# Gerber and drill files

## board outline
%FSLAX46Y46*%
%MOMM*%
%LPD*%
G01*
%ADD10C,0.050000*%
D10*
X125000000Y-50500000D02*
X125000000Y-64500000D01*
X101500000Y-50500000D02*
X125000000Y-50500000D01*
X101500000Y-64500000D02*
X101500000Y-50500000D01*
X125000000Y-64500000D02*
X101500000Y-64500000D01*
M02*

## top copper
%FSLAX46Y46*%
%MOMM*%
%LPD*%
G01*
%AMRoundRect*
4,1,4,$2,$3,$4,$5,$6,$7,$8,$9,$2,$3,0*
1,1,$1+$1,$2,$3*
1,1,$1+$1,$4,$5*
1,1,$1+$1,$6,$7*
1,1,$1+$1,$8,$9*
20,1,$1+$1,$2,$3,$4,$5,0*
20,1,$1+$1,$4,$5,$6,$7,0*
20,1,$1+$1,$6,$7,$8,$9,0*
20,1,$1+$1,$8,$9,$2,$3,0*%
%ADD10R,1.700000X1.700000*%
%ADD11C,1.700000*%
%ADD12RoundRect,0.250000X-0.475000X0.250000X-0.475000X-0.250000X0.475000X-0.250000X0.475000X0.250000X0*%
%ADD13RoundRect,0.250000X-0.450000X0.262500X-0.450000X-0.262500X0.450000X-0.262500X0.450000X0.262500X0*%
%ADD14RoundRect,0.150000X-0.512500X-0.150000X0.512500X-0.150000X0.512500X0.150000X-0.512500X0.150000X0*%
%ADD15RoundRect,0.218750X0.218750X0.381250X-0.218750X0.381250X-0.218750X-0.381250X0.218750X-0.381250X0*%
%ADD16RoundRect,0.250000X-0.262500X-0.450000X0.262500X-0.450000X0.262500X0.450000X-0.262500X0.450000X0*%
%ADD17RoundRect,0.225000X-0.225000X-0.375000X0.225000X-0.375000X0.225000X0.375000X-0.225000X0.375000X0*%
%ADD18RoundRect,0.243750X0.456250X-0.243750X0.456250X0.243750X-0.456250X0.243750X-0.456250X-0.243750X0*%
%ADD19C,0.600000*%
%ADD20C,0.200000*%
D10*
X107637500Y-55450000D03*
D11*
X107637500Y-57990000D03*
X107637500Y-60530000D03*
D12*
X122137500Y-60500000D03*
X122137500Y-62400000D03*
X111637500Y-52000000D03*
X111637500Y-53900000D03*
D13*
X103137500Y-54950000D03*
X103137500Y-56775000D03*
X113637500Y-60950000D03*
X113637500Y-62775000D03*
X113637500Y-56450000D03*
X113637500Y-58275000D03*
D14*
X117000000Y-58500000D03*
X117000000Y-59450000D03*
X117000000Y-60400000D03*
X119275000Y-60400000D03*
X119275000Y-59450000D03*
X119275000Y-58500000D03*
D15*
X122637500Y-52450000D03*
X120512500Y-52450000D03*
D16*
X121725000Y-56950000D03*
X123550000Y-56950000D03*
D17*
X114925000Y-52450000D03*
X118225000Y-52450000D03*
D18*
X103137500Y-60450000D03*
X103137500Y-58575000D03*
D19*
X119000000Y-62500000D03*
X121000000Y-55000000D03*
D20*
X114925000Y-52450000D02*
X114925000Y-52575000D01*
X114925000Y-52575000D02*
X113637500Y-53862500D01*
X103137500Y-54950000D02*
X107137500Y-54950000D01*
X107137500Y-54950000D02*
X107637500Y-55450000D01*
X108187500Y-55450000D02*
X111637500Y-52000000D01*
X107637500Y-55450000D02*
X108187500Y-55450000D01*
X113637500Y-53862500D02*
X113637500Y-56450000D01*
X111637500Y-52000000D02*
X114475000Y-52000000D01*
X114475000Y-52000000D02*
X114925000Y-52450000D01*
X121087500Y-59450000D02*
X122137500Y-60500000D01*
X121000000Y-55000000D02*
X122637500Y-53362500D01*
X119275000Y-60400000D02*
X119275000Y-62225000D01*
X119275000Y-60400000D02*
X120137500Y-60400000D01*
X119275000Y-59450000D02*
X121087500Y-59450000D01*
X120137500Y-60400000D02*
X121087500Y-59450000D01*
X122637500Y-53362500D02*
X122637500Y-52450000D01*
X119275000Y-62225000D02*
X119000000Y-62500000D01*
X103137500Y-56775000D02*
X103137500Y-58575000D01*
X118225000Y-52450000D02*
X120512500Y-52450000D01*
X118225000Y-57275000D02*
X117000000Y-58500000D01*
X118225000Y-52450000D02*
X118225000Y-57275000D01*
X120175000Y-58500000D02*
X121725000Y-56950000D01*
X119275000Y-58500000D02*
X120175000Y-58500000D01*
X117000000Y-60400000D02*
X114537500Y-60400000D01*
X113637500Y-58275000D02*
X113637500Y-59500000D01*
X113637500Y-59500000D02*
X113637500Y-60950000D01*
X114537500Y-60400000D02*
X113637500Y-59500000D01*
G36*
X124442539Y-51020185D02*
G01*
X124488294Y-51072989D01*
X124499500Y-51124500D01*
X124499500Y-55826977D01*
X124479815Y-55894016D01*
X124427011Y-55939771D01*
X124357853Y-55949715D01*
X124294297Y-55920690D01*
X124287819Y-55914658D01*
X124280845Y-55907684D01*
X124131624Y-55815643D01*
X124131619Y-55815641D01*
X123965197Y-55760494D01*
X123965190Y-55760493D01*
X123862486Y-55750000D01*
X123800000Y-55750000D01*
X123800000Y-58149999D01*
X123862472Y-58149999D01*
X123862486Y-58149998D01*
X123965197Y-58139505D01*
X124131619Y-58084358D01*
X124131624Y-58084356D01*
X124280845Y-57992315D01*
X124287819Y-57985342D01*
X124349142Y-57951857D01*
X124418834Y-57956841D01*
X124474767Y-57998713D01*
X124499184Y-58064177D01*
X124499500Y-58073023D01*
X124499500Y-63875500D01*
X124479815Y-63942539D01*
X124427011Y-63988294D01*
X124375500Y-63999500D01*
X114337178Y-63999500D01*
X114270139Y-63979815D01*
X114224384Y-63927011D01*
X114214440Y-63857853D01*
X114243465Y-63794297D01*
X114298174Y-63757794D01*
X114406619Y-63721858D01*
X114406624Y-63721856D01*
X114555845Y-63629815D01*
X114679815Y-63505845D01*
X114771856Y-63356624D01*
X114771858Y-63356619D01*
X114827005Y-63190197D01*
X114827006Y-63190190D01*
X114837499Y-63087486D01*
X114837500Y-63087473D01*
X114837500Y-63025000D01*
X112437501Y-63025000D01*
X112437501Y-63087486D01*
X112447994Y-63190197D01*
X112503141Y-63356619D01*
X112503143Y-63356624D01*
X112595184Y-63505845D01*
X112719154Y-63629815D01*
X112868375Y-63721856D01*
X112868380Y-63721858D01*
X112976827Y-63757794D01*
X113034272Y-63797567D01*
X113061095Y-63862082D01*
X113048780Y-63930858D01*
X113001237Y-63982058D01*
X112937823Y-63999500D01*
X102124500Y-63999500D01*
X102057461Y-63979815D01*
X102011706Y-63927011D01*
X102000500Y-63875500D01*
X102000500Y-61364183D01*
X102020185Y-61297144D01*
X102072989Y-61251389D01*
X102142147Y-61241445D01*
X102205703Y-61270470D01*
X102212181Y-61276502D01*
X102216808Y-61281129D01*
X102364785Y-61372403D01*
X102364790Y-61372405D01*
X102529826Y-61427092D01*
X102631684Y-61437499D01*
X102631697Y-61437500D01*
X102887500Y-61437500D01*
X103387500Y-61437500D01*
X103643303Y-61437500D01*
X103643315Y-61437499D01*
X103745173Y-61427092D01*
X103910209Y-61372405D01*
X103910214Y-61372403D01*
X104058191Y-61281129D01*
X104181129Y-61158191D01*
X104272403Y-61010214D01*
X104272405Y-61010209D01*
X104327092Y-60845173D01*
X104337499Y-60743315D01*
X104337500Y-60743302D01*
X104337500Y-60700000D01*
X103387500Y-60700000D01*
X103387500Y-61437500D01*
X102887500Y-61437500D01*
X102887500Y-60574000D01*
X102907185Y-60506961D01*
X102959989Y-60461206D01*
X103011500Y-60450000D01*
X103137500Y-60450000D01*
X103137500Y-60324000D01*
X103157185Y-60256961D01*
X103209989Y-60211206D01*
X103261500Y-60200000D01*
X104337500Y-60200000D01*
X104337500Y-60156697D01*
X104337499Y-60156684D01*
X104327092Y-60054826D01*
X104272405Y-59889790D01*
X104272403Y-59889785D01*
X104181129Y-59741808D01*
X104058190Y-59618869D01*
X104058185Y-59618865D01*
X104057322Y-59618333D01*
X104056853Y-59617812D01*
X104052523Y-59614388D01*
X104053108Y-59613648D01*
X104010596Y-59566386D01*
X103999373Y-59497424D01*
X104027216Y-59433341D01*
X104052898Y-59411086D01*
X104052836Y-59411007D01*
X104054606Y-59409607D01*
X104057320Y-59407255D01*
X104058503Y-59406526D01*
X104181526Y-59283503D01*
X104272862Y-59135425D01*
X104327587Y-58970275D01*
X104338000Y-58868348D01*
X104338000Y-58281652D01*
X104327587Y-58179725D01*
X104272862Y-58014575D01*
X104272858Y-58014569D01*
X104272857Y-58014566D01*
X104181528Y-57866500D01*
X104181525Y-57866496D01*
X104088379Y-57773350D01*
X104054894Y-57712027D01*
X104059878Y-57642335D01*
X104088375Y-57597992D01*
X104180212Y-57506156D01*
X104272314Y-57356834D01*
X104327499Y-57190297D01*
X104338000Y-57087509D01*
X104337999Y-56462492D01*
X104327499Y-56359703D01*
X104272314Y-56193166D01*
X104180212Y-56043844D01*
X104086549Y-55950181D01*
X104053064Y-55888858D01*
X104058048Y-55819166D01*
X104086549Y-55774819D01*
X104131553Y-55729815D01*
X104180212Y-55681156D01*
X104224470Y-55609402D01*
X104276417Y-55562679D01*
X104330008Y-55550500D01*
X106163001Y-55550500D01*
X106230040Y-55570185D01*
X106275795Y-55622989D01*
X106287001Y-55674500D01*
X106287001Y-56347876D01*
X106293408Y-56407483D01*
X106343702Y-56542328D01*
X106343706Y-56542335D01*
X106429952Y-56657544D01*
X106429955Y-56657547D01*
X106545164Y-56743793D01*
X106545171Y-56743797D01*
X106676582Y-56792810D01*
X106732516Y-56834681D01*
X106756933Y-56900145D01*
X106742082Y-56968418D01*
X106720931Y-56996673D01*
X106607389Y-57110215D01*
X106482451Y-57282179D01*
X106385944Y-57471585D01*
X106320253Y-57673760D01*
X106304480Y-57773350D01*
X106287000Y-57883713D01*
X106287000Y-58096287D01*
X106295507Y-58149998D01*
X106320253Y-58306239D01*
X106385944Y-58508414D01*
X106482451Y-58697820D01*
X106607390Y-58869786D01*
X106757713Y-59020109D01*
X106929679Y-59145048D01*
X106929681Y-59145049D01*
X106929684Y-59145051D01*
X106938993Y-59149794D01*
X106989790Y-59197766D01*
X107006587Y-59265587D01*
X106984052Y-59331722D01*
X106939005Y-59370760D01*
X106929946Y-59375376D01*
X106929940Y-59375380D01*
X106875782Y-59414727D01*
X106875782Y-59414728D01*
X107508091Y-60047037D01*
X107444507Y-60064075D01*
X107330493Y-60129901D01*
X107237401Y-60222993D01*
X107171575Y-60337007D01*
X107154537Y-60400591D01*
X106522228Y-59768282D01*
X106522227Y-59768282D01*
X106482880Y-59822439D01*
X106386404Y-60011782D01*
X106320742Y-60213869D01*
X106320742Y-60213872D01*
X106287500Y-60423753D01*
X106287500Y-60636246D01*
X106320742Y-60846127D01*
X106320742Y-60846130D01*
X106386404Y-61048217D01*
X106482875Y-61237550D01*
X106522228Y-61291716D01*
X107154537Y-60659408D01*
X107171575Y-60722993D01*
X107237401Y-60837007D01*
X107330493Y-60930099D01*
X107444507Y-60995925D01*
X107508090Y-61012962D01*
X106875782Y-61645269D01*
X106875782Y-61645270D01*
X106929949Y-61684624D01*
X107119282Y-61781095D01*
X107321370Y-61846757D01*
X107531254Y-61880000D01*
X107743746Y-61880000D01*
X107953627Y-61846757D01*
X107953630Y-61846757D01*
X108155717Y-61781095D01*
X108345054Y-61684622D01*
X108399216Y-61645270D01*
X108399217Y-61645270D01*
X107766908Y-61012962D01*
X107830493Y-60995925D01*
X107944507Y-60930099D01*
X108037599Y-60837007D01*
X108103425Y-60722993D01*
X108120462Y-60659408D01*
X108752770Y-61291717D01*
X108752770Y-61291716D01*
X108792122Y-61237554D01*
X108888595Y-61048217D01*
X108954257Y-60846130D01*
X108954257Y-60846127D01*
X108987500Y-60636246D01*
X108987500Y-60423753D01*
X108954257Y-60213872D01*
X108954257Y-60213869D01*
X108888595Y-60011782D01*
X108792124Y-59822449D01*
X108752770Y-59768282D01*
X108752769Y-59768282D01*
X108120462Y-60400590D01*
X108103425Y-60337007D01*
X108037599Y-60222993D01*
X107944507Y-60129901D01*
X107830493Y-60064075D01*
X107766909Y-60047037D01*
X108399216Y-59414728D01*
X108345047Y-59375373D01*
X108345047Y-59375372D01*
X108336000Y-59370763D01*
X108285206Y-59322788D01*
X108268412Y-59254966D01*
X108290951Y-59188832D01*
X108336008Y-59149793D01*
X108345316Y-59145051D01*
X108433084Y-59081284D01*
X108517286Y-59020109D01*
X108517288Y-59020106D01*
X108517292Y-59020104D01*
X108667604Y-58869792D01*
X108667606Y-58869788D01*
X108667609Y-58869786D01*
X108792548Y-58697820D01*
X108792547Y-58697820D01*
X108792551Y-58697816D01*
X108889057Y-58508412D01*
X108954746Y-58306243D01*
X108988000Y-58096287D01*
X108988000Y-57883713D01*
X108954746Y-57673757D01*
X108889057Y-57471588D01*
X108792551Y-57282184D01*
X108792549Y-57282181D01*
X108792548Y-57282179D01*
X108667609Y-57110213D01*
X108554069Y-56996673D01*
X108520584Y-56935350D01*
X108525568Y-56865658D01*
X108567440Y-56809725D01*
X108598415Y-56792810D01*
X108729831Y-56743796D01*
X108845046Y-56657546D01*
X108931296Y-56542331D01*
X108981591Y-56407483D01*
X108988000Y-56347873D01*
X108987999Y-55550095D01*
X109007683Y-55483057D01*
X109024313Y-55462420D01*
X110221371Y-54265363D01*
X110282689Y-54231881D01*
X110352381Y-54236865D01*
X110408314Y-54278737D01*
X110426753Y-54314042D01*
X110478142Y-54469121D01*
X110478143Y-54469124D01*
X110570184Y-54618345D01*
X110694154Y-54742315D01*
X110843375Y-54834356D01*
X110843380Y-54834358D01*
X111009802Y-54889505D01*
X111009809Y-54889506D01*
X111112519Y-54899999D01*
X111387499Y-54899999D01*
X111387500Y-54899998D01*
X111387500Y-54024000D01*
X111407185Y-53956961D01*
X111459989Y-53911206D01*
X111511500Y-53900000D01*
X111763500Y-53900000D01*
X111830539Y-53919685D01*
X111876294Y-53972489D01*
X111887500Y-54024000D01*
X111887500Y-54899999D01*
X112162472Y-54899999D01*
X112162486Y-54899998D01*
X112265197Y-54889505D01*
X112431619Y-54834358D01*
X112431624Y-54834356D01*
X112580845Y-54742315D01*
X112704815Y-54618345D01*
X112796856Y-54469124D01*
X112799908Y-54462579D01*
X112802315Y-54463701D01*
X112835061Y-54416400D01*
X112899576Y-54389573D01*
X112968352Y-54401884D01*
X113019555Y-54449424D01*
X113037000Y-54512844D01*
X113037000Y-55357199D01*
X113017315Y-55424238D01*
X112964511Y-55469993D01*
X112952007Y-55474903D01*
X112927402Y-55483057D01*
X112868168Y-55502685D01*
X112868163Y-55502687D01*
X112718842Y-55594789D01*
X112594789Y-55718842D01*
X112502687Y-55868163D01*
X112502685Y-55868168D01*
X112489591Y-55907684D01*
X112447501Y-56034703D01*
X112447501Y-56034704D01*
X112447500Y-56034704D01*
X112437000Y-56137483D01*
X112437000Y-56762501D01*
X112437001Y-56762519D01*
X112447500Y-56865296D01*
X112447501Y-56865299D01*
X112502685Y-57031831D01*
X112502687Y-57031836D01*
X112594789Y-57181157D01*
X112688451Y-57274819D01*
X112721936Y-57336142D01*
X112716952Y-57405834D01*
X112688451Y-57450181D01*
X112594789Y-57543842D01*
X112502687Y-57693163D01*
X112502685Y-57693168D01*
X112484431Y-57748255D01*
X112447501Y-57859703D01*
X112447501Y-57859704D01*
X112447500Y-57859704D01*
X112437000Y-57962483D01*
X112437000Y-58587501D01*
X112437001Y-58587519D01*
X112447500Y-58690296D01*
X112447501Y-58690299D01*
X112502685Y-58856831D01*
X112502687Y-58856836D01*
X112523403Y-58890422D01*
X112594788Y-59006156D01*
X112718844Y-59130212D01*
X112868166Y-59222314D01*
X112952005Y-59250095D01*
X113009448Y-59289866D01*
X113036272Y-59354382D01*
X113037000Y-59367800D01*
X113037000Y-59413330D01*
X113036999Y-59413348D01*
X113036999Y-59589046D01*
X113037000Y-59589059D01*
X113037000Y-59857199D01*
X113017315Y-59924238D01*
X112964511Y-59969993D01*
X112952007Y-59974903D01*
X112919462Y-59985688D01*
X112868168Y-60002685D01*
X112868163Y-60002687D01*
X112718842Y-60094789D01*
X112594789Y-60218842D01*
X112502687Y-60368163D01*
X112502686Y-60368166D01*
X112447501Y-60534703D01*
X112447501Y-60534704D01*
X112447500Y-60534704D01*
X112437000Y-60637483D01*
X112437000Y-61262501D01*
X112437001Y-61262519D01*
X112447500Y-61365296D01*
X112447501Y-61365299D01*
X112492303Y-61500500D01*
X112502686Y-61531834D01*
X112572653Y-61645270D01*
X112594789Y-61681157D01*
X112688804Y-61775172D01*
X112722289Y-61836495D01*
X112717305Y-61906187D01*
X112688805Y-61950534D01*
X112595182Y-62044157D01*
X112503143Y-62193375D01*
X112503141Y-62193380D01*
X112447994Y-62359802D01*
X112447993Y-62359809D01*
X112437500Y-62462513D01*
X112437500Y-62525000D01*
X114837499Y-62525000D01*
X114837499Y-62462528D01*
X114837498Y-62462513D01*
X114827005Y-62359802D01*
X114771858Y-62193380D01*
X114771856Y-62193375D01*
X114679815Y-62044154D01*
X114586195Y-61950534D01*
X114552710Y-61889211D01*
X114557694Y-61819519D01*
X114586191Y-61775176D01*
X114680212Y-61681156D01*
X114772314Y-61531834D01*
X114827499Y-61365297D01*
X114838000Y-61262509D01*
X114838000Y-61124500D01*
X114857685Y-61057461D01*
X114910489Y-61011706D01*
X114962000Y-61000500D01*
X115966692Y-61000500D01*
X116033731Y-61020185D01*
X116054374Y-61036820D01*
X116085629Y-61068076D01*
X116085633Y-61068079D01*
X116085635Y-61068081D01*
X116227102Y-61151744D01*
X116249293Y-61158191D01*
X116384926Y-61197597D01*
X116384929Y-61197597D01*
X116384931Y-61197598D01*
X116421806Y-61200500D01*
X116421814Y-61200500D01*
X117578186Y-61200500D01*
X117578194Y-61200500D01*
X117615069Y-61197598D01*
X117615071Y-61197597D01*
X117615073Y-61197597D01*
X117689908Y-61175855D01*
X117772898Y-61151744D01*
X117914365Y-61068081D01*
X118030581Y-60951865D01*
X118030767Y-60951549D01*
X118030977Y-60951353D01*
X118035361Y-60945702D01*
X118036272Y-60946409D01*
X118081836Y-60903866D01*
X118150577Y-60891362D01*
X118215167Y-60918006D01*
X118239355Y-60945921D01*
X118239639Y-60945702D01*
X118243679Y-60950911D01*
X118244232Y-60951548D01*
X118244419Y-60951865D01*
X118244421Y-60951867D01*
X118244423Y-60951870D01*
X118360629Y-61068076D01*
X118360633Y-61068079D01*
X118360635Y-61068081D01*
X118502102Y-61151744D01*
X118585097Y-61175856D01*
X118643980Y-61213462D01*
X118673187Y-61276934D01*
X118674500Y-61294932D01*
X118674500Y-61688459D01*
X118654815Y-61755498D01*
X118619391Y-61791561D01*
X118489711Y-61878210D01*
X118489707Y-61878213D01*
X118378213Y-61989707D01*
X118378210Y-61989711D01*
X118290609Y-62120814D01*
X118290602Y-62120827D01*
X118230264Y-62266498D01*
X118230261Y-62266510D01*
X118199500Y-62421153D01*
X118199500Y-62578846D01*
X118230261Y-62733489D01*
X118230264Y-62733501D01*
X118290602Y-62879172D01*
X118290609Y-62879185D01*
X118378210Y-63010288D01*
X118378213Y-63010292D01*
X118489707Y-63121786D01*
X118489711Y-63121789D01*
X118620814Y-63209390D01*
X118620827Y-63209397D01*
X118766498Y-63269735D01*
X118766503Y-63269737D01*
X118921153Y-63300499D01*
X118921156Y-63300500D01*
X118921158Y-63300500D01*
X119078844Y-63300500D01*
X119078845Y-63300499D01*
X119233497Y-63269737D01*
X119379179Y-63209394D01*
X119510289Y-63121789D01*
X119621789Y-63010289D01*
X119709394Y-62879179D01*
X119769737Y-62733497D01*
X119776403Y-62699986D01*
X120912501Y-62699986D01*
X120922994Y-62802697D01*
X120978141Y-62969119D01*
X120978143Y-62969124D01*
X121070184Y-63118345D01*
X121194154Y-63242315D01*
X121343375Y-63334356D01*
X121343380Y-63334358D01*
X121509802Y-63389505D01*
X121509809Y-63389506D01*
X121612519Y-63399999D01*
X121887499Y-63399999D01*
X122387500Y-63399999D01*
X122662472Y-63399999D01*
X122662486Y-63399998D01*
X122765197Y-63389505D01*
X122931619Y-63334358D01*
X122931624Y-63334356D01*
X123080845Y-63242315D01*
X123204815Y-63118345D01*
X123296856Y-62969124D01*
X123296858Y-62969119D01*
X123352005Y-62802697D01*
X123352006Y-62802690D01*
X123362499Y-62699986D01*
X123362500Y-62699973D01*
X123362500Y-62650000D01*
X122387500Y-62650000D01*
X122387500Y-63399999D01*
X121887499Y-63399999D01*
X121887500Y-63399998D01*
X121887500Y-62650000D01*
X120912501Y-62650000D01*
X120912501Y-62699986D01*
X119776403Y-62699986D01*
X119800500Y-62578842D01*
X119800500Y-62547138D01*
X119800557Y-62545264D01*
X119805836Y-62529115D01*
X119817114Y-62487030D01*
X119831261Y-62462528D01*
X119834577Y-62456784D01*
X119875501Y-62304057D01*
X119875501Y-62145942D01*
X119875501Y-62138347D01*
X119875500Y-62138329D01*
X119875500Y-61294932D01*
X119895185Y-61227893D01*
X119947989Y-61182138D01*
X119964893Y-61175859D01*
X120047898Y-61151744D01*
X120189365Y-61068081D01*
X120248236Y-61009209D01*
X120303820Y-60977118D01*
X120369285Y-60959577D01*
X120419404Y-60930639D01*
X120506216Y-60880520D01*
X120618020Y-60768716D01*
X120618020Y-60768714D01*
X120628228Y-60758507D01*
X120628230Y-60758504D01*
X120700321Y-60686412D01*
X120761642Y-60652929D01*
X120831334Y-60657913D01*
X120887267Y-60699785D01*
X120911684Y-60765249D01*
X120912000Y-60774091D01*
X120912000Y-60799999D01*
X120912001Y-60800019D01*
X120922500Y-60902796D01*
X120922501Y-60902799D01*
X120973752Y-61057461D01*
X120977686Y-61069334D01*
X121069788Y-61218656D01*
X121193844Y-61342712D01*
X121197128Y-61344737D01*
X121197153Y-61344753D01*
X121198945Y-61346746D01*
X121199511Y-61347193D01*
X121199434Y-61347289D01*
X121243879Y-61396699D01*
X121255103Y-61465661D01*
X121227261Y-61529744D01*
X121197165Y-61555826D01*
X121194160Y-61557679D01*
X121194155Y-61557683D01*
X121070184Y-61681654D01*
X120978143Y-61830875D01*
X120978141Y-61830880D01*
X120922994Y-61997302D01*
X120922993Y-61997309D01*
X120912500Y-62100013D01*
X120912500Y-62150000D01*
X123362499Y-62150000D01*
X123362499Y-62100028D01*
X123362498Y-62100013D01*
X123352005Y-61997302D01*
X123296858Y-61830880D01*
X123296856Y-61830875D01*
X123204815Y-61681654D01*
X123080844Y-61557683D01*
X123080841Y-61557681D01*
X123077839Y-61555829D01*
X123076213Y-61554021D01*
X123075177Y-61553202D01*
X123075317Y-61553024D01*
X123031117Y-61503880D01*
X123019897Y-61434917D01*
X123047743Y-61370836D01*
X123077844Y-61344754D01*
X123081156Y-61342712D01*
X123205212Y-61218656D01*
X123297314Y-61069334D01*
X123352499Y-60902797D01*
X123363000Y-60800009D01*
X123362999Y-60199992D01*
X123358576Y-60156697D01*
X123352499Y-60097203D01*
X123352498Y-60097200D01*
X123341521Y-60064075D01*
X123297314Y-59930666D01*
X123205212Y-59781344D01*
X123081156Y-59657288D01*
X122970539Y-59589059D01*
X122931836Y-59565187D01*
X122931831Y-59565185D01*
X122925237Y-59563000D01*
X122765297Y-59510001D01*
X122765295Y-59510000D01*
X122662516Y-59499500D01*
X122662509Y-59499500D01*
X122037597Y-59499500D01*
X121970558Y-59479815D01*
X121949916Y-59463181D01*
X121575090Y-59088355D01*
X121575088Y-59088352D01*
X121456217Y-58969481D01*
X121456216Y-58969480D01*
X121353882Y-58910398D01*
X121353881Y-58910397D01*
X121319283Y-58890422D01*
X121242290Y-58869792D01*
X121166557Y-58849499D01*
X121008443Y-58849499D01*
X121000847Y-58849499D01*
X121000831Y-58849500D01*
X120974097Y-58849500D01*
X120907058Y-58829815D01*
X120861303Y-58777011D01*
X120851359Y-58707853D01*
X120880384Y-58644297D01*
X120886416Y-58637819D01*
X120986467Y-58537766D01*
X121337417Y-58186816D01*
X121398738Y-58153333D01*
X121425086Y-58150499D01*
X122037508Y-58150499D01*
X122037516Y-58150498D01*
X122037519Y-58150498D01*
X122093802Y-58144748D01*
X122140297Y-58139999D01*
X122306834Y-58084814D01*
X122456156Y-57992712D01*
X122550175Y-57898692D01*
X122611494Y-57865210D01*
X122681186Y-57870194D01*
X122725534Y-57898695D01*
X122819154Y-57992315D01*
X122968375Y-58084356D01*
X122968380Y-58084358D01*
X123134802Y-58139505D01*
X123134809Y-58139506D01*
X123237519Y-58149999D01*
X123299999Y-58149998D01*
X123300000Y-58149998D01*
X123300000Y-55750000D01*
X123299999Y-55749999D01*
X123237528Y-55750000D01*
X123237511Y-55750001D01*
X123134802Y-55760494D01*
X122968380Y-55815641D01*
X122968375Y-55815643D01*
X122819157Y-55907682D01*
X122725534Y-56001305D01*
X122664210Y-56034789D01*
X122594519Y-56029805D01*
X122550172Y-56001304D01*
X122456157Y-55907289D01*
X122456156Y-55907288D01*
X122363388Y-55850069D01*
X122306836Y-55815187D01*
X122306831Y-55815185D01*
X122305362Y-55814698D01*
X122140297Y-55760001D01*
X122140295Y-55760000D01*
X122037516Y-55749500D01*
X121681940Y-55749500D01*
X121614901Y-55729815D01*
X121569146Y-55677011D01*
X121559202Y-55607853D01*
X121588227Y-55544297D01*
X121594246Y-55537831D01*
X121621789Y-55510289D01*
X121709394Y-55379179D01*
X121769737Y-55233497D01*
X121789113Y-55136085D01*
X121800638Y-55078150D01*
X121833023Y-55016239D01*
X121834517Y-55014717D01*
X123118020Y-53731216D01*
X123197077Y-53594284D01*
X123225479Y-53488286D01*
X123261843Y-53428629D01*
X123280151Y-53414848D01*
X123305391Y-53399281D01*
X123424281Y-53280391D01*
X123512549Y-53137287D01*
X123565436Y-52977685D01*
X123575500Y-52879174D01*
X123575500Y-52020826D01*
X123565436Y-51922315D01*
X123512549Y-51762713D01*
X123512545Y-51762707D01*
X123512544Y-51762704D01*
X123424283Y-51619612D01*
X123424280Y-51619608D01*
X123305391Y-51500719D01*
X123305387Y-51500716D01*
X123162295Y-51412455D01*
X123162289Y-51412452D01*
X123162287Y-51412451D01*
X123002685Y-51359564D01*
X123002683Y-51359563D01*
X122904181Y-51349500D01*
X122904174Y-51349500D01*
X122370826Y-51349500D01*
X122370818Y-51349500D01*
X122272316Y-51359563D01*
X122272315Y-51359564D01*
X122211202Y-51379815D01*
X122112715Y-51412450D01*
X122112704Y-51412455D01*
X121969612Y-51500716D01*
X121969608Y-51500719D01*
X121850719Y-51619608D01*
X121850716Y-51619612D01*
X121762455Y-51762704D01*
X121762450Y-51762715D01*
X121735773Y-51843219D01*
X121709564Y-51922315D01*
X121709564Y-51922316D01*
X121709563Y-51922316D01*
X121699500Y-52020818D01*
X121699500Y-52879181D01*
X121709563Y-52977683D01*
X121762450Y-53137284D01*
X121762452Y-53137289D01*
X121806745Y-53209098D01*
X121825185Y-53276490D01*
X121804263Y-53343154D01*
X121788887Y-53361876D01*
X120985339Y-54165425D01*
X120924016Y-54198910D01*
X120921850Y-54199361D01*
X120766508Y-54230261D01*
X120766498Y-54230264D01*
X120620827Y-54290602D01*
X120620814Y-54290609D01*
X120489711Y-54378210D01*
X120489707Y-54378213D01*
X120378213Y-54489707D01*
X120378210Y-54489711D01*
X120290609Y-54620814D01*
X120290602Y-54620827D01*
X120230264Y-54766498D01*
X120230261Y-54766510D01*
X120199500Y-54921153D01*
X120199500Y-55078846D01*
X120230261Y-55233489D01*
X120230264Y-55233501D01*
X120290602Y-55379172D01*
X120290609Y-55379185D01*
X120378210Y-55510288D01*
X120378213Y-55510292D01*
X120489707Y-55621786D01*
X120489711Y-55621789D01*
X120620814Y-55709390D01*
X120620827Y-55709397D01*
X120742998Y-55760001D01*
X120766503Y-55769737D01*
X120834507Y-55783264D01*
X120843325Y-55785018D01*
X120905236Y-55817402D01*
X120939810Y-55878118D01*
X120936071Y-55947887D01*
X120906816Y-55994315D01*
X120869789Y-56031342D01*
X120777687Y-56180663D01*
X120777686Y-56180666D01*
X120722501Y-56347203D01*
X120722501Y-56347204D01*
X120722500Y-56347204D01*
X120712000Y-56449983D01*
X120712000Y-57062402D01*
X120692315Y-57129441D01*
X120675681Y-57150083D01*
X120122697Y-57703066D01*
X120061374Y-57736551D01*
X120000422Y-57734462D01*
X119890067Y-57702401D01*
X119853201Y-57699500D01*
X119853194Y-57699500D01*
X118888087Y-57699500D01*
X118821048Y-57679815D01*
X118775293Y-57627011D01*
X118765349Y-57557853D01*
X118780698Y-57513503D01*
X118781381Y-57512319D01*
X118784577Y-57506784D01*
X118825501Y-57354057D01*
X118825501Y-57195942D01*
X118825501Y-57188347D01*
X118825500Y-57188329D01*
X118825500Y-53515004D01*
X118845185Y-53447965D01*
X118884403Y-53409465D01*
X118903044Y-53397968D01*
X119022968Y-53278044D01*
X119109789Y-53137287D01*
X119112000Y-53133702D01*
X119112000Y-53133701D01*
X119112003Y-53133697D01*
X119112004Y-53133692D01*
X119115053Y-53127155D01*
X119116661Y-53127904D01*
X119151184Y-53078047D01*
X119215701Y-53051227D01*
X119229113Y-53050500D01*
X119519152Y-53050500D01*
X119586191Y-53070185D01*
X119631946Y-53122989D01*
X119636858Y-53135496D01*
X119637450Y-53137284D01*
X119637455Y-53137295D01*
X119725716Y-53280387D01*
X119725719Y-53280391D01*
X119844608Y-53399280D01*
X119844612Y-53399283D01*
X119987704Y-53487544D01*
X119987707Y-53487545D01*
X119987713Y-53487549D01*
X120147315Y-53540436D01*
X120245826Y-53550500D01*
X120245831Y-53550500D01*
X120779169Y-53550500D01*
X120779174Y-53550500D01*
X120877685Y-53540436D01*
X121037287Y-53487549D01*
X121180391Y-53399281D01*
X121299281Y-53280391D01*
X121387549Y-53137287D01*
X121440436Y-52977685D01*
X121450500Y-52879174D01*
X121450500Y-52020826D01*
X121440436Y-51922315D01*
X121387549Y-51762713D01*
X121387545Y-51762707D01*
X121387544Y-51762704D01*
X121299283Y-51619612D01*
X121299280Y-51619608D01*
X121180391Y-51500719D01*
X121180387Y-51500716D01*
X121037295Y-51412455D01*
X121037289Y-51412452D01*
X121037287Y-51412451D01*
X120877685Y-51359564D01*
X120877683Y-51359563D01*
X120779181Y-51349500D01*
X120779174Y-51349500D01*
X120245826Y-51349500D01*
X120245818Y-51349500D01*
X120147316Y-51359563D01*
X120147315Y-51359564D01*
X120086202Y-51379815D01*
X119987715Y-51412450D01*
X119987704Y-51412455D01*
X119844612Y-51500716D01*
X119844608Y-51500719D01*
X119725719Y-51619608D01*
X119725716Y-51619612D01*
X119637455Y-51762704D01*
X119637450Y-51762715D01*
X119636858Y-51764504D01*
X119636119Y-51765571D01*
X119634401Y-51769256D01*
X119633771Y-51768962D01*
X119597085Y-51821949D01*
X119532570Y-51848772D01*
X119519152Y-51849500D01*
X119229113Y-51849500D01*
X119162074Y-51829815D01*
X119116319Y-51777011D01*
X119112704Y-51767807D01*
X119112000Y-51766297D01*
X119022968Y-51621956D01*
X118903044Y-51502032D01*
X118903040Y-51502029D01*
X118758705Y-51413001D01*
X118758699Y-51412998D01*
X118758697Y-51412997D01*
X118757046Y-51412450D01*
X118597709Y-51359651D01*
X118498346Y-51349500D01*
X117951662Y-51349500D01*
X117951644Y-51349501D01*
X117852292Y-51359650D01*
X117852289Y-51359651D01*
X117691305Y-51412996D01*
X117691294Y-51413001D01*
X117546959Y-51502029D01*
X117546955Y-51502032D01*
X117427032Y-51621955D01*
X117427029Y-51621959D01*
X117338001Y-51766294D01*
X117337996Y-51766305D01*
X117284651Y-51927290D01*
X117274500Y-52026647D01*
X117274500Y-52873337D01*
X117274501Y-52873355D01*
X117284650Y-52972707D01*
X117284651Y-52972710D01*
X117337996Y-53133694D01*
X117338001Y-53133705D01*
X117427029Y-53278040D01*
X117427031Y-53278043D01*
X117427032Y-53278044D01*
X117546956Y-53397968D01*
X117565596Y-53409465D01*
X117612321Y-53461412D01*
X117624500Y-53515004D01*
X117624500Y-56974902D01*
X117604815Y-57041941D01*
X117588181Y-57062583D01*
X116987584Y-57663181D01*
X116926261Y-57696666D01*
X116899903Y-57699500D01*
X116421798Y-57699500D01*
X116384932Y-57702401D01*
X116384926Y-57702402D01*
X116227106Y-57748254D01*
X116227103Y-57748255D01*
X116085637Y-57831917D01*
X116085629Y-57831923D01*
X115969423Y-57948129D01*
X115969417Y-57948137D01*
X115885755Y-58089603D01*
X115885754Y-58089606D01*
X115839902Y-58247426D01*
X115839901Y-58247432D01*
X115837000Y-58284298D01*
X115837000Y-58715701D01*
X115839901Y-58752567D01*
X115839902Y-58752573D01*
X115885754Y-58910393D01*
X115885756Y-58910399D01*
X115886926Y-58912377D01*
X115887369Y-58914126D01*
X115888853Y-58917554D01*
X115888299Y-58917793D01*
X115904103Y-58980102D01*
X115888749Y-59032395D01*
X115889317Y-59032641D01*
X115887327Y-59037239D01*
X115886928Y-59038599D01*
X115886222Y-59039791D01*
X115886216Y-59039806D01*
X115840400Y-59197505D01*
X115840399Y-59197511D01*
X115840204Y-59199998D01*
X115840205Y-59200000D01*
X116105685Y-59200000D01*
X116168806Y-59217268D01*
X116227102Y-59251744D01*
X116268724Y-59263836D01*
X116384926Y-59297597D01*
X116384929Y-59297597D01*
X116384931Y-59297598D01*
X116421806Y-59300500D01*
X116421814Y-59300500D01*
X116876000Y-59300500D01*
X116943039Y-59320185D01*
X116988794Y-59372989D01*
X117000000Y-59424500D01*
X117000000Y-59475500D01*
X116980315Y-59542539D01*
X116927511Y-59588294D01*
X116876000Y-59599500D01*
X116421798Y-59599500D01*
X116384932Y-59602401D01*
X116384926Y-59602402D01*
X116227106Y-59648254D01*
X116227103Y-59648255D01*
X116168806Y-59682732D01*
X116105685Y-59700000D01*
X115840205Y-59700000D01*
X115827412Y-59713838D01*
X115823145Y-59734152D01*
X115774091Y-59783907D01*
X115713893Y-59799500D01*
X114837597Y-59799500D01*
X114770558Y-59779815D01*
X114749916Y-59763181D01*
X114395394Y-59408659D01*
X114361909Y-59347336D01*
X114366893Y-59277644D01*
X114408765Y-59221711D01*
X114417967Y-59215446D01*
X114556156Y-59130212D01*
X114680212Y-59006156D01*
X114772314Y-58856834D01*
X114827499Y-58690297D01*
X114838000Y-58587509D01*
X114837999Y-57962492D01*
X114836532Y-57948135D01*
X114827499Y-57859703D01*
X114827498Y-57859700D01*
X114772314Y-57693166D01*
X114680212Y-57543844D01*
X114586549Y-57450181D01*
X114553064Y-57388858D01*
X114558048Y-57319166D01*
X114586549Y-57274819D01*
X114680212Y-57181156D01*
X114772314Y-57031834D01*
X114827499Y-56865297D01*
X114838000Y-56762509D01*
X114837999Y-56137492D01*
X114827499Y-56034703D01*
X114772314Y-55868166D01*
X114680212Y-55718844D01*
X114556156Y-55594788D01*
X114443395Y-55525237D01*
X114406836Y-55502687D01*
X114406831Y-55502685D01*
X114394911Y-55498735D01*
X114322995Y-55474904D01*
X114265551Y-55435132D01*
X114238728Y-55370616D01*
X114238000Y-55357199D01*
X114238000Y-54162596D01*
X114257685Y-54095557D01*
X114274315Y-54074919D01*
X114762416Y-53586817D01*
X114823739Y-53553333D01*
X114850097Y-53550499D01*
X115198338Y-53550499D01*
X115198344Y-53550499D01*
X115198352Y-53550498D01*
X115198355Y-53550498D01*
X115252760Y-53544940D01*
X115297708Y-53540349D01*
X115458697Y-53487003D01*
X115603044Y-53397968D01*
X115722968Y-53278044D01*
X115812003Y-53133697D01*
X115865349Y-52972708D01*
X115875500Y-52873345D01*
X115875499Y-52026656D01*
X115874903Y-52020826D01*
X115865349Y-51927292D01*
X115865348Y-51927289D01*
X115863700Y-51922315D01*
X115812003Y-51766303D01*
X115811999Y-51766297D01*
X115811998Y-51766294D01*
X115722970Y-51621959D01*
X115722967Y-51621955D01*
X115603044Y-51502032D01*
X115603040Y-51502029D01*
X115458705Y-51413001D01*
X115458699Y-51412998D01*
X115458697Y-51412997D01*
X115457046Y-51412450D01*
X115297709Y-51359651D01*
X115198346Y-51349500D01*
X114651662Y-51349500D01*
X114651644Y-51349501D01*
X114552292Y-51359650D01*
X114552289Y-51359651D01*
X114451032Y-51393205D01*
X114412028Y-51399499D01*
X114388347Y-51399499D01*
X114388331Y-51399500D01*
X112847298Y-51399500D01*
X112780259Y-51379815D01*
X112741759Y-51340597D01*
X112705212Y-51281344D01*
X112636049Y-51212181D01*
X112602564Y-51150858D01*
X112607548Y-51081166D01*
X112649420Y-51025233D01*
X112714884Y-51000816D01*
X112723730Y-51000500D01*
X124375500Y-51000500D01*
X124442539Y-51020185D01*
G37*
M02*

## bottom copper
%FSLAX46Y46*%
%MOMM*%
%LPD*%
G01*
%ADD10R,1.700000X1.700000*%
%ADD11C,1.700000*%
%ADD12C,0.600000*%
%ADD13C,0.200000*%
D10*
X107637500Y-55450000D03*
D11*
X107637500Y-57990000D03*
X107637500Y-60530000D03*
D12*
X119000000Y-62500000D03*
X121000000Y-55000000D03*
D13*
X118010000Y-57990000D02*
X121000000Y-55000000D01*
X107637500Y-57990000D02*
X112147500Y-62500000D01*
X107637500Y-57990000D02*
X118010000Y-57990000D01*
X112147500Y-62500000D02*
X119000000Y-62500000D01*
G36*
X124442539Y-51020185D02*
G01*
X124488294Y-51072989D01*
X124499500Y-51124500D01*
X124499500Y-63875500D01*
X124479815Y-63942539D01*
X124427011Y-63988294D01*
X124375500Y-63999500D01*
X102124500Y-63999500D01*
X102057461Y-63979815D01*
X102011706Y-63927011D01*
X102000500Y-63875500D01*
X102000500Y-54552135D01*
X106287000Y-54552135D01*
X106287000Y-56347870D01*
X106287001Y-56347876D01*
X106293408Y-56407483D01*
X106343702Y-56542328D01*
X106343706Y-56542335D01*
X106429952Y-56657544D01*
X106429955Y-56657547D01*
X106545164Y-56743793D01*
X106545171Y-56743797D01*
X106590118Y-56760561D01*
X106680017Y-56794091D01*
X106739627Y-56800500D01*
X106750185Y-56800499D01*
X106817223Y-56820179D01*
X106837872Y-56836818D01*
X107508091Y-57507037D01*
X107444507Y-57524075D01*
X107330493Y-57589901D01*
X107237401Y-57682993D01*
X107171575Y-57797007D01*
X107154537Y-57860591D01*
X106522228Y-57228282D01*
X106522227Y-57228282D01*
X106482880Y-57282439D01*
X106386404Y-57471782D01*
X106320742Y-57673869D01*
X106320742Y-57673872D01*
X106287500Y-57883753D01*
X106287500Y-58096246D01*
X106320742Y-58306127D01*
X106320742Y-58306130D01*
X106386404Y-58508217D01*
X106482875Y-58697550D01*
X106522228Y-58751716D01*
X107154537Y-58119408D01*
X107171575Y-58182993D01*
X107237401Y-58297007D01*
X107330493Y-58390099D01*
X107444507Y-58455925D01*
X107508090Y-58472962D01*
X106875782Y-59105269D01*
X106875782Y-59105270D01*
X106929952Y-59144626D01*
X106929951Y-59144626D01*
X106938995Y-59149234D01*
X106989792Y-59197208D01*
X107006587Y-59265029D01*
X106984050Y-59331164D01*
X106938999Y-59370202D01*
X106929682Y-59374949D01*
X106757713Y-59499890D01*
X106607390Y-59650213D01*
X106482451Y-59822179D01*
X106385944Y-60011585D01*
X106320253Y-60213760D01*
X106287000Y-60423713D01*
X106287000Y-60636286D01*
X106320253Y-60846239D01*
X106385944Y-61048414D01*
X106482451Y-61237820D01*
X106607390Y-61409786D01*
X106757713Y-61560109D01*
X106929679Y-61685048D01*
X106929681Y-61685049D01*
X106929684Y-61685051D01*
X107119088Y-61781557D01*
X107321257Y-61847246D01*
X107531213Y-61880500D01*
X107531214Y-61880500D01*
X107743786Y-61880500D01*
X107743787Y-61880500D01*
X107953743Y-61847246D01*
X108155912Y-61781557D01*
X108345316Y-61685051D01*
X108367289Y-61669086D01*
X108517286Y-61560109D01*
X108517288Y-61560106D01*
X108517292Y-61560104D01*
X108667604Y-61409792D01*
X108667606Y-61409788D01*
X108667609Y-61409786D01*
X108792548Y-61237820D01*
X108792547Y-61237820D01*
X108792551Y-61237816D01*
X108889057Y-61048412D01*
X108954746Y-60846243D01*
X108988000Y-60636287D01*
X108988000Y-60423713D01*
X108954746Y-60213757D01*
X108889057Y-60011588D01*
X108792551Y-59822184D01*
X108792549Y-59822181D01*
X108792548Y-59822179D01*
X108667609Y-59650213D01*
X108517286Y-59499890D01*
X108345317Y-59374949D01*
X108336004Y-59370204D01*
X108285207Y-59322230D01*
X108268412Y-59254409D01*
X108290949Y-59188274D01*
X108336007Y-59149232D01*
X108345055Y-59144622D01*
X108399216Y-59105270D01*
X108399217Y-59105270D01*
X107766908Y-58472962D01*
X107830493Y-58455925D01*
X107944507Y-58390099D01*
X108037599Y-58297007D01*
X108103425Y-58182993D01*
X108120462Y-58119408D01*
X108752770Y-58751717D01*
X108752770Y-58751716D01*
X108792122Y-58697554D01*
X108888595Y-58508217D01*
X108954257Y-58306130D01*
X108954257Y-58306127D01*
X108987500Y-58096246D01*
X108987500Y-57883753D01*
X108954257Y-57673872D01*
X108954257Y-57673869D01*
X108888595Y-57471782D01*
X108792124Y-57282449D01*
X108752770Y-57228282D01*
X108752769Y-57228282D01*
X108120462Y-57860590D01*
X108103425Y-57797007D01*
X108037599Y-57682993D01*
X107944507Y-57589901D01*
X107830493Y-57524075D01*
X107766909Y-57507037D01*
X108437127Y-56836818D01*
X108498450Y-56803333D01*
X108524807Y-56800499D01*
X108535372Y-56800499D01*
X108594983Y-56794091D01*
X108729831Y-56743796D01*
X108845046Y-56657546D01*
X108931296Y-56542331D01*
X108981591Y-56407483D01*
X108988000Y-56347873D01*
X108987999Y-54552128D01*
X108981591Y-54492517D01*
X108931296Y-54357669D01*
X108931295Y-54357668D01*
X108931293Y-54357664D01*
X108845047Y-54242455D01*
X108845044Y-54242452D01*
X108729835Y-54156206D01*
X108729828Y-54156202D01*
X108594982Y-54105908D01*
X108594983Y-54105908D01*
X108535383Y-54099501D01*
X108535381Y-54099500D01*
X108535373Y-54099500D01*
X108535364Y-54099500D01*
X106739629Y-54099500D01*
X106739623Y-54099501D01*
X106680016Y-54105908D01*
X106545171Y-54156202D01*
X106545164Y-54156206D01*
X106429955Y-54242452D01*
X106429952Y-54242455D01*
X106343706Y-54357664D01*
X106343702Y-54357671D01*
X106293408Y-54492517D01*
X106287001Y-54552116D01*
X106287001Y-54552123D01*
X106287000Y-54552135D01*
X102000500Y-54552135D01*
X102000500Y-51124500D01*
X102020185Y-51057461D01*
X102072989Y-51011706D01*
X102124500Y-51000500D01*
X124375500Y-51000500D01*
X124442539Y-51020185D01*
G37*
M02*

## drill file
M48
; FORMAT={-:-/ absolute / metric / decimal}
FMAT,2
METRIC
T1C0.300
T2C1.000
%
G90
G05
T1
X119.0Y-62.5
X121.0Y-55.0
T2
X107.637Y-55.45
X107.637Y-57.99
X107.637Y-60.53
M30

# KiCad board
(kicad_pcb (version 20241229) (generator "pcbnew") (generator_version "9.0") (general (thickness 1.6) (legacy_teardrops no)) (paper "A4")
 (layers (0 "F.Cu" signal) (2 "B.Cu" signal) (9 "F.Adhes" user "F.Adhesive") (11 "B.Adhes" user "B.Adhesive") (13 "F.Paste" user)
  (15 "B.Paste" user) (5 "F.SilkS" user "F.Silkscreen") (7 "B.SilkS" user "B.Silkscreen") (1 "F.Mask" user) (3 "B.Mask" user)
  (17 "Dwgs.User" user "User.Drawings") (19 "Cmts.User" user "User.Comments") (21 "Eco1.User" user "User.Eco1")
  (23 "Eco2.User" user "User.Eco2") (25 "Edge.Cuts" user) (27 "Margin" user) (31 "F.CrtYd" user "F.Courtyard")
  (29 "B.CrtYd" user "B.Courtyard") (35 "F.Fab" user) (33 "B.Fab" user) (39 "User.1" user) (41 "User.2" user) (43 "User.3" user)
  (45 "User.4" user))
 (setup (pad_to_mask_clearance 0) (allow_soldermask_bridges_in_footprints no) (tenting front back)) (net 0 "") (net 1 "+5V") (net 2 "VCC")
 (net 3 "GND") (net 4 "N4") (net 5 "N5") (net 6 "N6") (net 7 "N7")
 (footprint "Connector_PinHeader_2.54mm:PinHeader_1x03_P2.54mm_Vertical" (layer "F.Cu") (at 107.6375 55.45)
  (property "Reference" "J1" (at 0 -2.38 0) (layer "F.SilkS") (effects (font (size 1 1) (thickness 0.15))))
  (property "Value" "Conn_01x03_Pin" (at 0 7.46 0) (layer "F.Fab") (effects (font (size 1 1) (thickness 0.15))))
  (pad "1" thru_hole rect (at 0 0) (size 1.7 1.7) (drill 1) (layers "*.Cu" "*.Mask") (remove_unused_layers no) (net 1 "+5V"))
  (pad "2" thru_hole circle (at 0 2.54) (size 1.7 1.7) (drill 1) (layers "*.Cu" "*.Mask") (remove_unused_layers no) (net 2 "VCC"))
  (pad "3" thru_hole circle (at 0 5.08) (size 1.7 1.7) (drill 1) (layers "*.Cu" "*.Mask") (remove_unused_layers no) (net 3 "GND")))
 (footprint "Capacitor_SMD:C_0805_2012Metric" (layer "F.Cu") (at 122.1375 61.45 -90)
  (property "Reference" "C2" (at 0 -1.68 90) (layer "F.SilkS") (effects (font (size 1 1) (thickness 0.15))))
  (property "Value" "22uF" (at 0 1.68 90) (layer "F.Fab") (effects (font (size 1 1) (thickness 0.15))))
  (pad "1" smd roundrect (at -0.95 0 270) (size 1 1.45) (layers "F.Cu" "F.Mask" "F.Paste") (roundrect_rratio 0.25) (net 2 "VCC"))
  (pad "2" smd roundrect (at 0.95 0 270) (size 1 1.45) (layers "F.Cu" "F.Mask" "F.Paste") (roundrect_rratio 0.25) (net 3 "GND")))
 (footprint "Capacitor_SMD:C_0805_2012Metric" (layer "F.Cu") (at 111.6375 52.95 -90)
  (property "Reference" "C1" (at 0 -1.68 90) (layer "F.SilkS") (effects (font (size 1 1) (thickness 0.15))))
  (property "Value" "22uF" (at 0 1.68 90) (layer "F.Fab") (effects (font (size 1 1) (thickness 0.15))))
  (pad "1" smd roundrect (at -0.95 0 270) (size 1 1.45) (layers "F.Cu" "F.Mask" "F.Paste") (roundrect_rratio 0.25) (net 1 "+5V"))
  (pad "2" smd roundrect (at 0.95 0 270) (size 1 1.45) (layers "F.Cu" "F.Mask" "F.Paste") (roundrect_rratio 0.25) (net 3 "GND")))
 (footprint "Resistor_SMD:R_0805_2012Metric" (layer "F.Cu") (at 103.1375 55.8625 -90)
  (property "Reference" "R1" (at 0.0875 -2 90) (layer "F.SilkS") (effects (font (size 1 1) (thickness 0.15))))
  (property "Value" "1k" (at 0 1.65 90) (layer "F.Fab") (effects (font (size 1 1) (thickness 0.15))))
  (pad "1" smd roundrect (at -0.9125 0 270) (size 1.025 1.4) (layers "F.Cu" "F.Mask" "F.Paste") (roundrect_rratio 0.243902) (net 1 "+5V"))
  (pad "2" smd roundrect (at 0.9125 0 270) (size 1.025 1.4) (layers "F.Cu" "F.Mask" "F.Paste") (roundrect_rratio 0.243902) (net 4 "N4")))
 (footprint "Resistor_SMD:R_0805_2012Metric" (layer "F.Cu") (at 113.6375 61.8625 -90)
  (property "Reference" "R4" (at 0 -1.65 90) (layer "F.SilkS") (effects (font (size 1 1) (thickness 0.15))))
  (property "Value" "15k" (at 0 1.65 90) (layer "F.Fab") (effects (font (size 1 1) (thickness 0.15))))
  (pad "1" smd roundrect (at -0.9125 0 270) (size 1.025 1.4) (layers "F.Cu" "F.Mask" "F.Paste") (roundrect_rratio 0.243902) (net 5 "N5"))
  (pad "2" smd roundrect (at 0.9125 0 270) (size 1.025 1.4) (layers "F.Cu" "F.Mask" "F.Paste") (roundrect_rratio 0.243902) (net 3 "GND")))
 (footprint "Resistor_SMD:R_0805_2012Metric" (layer "F.Cu") (at 113.6375 57.3625 -90)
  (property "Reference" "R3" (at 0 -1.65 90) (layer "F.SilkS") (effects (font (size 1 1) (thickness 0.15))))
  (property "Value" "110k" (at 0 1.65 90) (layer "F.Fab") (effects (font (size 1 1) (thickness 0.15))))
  (pad "1" smd roundrect (at -0.9125 0 270) (size 1.025 1.4) (layers "F.Cu" "F.Mask" "F.Paste") (roundrect_rratio 0.243902) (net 1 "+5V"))
  (pad "2" smd roundrect (at 0.9125 0 270) (size 1.025 1.4) (layers "F.Cu" "F.Mask" "F.Paste") (roundrect_rratio 0.243902) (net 5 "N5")))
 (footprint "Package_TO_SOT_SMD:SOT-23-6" (layer "F.Cu") (at 118.1375 59.45)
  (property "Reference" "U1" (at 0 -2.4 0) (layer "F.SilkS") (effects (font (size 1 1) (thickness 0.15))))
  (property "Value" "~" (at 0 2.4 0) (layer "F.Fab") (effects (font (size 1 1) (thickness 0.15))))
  (pad "1" smd roundrect (at -1.1375 -0.95) (size 1.325 0.6) (layers "F.Cu" "F.Mask" "F.Paste") (roundrect_rratio 0.25) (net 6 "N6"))
  (pad "2" smd roundrect (at -1.1375 0) (size 1.325 0.6) (layers "F.Cu" "F.Mask" "F.Paste") (roundrect_rratio 0.25) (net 3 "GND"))
  (pad "3" smd roundrect (at -1.1375 0.95) (size 1.325 0.6) (layers "F.Cu" "F.Mask" "F.Paste") (roundrect_rratio 0.25) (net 5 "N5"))
  (pad "4" smd roundrect (at 1.1375 0.95) (size 1.325 0.6) (layers "F.Cu" "F.Mask" "F.Paste") (roundrect_rratio 0.25) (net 2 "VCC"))
  (pad "5" smd roundrect (at 1.1375 0) (size 1.325 0.6) (layers "F.Cu" "F.Mask" "F.Paste") (roundrect_rratio 0.25) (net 2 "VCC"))
  (pad "6" smd roundrect (at 1.1375 -0.95) (size 1.325 0.6) (layers "F.Cu" "F.Mask" "F.Paste") (roundrect_rratio 0.25) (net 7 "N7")))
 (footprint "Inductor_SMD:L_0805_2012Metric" (layer "F.Cu") (at 121.575 52.45 180)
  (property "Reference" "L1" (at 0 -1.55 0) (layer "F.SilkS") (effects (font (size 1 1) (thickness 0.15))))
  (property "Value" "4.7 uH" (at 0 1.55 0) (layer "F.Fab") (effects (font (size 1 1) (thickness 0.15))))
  (pad "1" smd roundrect (at -1.0625 0 180) (size 0.875 1.2) (layers "F.Cu" "F.Mask" "F.Paste") (roundrect_rratio 0.25) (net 2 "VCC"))
  (pad "2" smd roundrect (at 1.0625 0 180) (size 0.875 1.2) (layers "F.Cu" "F.Mask" "F.Paste") (roundrect_rratio 0.25) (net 6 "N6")))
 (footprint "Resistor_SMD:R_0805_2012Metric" (layer "F.Cu") (at 122.6375 56.95)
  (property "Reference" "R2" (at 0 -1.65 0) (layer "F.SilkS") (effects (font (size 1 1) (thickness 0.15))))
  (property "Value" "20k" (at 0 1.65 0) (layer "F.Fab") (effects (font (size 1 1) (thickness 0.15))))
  (pad "1" smd roundrect (at -0.9125 0) (size 1.025 1.4) (layers "F.Cu" "F.Mask" "F.Paste") (roundrect_rratio 0.243902) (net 7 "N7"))
  (pad "2" smd roundrect (at 0.9125 0) (size 1.025 1.4) (layers "F.Cu" "F.Mask" "F.Paste") (roundrect_rratio 0.243902) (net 3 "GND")))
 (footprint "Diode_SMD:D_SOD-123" (layer "F.Cu") (at 116.575 52.45)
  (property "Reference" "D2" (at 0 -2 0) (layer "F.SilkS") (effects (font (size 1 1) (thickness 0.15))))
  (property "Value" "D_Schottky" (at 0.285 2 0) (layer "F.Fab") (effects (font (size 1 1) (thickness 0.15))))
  (pad "1" smd roundrect (at -1.65 0) (size 0.9 1.2) (layers "F.Cu" "F.Mask" "F.Paste") (roundrect_rratio 0.25) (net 1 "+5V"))
  (pad "2" smd roundrect (at 1.65 0) (size 0.9 1.2) (layers "F.Cu" "F.Mask" "F.Paste") (roundrect_rratio 0.25) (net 6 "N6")))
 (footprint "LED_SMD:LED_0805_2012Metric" (layer "F.Cu") (at 103.1375 59.5125 90)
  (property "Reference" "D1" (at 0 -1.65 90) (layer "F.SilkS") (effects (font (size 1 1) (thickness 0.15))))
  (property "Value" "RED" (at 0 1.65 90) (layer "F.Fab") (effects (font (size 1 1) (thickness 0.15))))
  (pad "1" smd roundrect (at -0.9375 0 90) (size 0.975 1.4) (layers "F.Cu" "F.Mask" "F.Paste") (roundrect_rratio 0.25) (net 3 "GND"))
  (pad "2" smd roundrect (at 0.9375 0 90) (size 0.975 1.4) (layers "F.Cu" "F.Mask" "F.Paste") (roundrect_rratio 0.25) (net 4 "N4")))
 (gr_line (start 125 50.5) (end 125 64.5) (stroke (width 0.05) (type default)) (layer "Edge.Cuts"))
 (gr_line (start 101.5 50.5) (end 125 50.5) (stroke (width 0.05) (type default)) (layer "Edge.Cuts"))
 (gr_line (start 101.5 64.5) (end 101.5 50.5) (stroke (width 0.05) (type default)) (layer "Edge.Cuts"))
 (gr_line (start 125 64.5) (end 101.5 64.5) (stroke (width 0.05) (type default)) (layer "Edge.Cuts"))
 (segment (start 114.925 52.45) (end 114.925 52.575) (width 0.2) (layer "F.Cu") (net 1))
 (segment (start 114.925 52.575) (end 113.6375 53.8625) (width 0.2) (layer "F.Cu") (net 1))
 (segment (start 103.1375 54.95) (end 107.1375 54.95) (width 0.2) (layer "F.Cu") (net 1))
 (segment (start 107.1375 54.95) (end 107.6375 55.45) (width 0.2) (layer "F.Cu") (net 1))
 (segment (start 108.1875 55.45) (end 111.6375 52) (width 0.2) (layer "F.Cu") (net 1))
 (segment (start 107.6375 55.45) (end 108.1875 55.45) (width 0.2) (layer "F.Cu") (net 1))
 (segment (start 113.6375 53.8625) (end 113.6375 56.45) (width 0.2) (layer "F.Cu") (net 1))
 (segment (start 111.6375 52) (end 114.475 52) (width 0.2) (layer "F.Cu") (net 1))
 (segment (start 114.475 52) (end 114.925 52.45) (width 0.2) (layer "F.Cu") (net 1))
 (segment (start 121.0875 59.45) (end 122.1375 60.5) (width 0.2) (layer "F.Cu") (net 2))
 (segment (start 121 55) (end 122.6375 53.3625) (width 0.2) (layer "F.Cu") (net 2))
 (segment (start 119.275 60.4) (end 119.275 62.225) (width 0.2) (layer "F.Cu") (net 2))
 (segment (start 119.275 60.4) (end 120.1375 60.4) (width 0.2) (layer "F.Cu") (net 2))
 (segment (start 119.275 59.45) (end 121.0875 59.45) (width 0.2) (layer "F.Cu") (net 2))
 (segment (start 120.1375 60.4) (end 121.0875 59.45) (width 0.2) (layer "F.Cu") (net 2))
 (segment (start 122.6375 53.3625) (end 122.6375 52.45) (width 0.2) (layer "F.Cu") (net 2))
 (segment (start 119.275 62.225) (end 119 62.5) (width 0.2) (layer "F.Cu") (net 2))
 (via (at 119 62.5) (size 0.6) (drill 0.3) (layers "F.Cu" "B.Cu") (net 2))
 (via (at 121 55) (size 0.6) (drill 0.3) (layers "F.Cu" "B.Cu") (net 2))
 (segment (start 118.01 57.99) (end 121 55) (width 0.2) (layer "B.Cu") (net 2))
 (segment (start 107.6375 57.99) (end 112.1475 62.5) (width 0.2) (layer "B.Cu") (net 2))
 (segment (start 107.6375 57.99) (end 118.01 57.99) (width 0.2) (layer "B.Cu") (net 2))
 (segment (start 112.1475 62.5) (end 119 62.5) (width 0.2) (layer "B.Cu") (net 2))
 (segment (start 103.1375 56.775) (end 103.1375 58.575) (width 0.2) (layer "F.Cu") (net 4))
 (segment (start 118.225 52.45) (end 120.5125 52.45) (width 0.2) (layer "F.Cu") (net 6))
 (segment (start 118.225 57.275) (end 117 58.5) (width 0.2) (layer "F.Cu") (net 6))
 (segment (start 118.225 52.45) (end 118.225 57.275) (width 0.2) (layer "F.Cu") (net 6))
 (segment (start 120.175 58.5) (end 121.725 56.95) (width 0.2) (layer "F.Cu") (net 7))
 (segment (start 119.275 58.5) (end 120.175 58.5) (width 0.2) (layer "F.Cu") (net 7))
 (segment (start 117 60.4) (end 114.5375 60.4) (width 0.2) (layer "F.Cu") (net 5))
 (segment (start 113.6375 58.275) (end 113.6375 59.5) (width 0.2) (layer "F.Cu") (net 5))
 (segment (start 113.6375 59.5) (end 113.6375 60.95) (width 0.2) (layer "F.Cu") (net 5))
 (segment (start 114.5375 60.4) (end 113.6375 59.5) (width 0.2) (layer "F.Cu") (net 5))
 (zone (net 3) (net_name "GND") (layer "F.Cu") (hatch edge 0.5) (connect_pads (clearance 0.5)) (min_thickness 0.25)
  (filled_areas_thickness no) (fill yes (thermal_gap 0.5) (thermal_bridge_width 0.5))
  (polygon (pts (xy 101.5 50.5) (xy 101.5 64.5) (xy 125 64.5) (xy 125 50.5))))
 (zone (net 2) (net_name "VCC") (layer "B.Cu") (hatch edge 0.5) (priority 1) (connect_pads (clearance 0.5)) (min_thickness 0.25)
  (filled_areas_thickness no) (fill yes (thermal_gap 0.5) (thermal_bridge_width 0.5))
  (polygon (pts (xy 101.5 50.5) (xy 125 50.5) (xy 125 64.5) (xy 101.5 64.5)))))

